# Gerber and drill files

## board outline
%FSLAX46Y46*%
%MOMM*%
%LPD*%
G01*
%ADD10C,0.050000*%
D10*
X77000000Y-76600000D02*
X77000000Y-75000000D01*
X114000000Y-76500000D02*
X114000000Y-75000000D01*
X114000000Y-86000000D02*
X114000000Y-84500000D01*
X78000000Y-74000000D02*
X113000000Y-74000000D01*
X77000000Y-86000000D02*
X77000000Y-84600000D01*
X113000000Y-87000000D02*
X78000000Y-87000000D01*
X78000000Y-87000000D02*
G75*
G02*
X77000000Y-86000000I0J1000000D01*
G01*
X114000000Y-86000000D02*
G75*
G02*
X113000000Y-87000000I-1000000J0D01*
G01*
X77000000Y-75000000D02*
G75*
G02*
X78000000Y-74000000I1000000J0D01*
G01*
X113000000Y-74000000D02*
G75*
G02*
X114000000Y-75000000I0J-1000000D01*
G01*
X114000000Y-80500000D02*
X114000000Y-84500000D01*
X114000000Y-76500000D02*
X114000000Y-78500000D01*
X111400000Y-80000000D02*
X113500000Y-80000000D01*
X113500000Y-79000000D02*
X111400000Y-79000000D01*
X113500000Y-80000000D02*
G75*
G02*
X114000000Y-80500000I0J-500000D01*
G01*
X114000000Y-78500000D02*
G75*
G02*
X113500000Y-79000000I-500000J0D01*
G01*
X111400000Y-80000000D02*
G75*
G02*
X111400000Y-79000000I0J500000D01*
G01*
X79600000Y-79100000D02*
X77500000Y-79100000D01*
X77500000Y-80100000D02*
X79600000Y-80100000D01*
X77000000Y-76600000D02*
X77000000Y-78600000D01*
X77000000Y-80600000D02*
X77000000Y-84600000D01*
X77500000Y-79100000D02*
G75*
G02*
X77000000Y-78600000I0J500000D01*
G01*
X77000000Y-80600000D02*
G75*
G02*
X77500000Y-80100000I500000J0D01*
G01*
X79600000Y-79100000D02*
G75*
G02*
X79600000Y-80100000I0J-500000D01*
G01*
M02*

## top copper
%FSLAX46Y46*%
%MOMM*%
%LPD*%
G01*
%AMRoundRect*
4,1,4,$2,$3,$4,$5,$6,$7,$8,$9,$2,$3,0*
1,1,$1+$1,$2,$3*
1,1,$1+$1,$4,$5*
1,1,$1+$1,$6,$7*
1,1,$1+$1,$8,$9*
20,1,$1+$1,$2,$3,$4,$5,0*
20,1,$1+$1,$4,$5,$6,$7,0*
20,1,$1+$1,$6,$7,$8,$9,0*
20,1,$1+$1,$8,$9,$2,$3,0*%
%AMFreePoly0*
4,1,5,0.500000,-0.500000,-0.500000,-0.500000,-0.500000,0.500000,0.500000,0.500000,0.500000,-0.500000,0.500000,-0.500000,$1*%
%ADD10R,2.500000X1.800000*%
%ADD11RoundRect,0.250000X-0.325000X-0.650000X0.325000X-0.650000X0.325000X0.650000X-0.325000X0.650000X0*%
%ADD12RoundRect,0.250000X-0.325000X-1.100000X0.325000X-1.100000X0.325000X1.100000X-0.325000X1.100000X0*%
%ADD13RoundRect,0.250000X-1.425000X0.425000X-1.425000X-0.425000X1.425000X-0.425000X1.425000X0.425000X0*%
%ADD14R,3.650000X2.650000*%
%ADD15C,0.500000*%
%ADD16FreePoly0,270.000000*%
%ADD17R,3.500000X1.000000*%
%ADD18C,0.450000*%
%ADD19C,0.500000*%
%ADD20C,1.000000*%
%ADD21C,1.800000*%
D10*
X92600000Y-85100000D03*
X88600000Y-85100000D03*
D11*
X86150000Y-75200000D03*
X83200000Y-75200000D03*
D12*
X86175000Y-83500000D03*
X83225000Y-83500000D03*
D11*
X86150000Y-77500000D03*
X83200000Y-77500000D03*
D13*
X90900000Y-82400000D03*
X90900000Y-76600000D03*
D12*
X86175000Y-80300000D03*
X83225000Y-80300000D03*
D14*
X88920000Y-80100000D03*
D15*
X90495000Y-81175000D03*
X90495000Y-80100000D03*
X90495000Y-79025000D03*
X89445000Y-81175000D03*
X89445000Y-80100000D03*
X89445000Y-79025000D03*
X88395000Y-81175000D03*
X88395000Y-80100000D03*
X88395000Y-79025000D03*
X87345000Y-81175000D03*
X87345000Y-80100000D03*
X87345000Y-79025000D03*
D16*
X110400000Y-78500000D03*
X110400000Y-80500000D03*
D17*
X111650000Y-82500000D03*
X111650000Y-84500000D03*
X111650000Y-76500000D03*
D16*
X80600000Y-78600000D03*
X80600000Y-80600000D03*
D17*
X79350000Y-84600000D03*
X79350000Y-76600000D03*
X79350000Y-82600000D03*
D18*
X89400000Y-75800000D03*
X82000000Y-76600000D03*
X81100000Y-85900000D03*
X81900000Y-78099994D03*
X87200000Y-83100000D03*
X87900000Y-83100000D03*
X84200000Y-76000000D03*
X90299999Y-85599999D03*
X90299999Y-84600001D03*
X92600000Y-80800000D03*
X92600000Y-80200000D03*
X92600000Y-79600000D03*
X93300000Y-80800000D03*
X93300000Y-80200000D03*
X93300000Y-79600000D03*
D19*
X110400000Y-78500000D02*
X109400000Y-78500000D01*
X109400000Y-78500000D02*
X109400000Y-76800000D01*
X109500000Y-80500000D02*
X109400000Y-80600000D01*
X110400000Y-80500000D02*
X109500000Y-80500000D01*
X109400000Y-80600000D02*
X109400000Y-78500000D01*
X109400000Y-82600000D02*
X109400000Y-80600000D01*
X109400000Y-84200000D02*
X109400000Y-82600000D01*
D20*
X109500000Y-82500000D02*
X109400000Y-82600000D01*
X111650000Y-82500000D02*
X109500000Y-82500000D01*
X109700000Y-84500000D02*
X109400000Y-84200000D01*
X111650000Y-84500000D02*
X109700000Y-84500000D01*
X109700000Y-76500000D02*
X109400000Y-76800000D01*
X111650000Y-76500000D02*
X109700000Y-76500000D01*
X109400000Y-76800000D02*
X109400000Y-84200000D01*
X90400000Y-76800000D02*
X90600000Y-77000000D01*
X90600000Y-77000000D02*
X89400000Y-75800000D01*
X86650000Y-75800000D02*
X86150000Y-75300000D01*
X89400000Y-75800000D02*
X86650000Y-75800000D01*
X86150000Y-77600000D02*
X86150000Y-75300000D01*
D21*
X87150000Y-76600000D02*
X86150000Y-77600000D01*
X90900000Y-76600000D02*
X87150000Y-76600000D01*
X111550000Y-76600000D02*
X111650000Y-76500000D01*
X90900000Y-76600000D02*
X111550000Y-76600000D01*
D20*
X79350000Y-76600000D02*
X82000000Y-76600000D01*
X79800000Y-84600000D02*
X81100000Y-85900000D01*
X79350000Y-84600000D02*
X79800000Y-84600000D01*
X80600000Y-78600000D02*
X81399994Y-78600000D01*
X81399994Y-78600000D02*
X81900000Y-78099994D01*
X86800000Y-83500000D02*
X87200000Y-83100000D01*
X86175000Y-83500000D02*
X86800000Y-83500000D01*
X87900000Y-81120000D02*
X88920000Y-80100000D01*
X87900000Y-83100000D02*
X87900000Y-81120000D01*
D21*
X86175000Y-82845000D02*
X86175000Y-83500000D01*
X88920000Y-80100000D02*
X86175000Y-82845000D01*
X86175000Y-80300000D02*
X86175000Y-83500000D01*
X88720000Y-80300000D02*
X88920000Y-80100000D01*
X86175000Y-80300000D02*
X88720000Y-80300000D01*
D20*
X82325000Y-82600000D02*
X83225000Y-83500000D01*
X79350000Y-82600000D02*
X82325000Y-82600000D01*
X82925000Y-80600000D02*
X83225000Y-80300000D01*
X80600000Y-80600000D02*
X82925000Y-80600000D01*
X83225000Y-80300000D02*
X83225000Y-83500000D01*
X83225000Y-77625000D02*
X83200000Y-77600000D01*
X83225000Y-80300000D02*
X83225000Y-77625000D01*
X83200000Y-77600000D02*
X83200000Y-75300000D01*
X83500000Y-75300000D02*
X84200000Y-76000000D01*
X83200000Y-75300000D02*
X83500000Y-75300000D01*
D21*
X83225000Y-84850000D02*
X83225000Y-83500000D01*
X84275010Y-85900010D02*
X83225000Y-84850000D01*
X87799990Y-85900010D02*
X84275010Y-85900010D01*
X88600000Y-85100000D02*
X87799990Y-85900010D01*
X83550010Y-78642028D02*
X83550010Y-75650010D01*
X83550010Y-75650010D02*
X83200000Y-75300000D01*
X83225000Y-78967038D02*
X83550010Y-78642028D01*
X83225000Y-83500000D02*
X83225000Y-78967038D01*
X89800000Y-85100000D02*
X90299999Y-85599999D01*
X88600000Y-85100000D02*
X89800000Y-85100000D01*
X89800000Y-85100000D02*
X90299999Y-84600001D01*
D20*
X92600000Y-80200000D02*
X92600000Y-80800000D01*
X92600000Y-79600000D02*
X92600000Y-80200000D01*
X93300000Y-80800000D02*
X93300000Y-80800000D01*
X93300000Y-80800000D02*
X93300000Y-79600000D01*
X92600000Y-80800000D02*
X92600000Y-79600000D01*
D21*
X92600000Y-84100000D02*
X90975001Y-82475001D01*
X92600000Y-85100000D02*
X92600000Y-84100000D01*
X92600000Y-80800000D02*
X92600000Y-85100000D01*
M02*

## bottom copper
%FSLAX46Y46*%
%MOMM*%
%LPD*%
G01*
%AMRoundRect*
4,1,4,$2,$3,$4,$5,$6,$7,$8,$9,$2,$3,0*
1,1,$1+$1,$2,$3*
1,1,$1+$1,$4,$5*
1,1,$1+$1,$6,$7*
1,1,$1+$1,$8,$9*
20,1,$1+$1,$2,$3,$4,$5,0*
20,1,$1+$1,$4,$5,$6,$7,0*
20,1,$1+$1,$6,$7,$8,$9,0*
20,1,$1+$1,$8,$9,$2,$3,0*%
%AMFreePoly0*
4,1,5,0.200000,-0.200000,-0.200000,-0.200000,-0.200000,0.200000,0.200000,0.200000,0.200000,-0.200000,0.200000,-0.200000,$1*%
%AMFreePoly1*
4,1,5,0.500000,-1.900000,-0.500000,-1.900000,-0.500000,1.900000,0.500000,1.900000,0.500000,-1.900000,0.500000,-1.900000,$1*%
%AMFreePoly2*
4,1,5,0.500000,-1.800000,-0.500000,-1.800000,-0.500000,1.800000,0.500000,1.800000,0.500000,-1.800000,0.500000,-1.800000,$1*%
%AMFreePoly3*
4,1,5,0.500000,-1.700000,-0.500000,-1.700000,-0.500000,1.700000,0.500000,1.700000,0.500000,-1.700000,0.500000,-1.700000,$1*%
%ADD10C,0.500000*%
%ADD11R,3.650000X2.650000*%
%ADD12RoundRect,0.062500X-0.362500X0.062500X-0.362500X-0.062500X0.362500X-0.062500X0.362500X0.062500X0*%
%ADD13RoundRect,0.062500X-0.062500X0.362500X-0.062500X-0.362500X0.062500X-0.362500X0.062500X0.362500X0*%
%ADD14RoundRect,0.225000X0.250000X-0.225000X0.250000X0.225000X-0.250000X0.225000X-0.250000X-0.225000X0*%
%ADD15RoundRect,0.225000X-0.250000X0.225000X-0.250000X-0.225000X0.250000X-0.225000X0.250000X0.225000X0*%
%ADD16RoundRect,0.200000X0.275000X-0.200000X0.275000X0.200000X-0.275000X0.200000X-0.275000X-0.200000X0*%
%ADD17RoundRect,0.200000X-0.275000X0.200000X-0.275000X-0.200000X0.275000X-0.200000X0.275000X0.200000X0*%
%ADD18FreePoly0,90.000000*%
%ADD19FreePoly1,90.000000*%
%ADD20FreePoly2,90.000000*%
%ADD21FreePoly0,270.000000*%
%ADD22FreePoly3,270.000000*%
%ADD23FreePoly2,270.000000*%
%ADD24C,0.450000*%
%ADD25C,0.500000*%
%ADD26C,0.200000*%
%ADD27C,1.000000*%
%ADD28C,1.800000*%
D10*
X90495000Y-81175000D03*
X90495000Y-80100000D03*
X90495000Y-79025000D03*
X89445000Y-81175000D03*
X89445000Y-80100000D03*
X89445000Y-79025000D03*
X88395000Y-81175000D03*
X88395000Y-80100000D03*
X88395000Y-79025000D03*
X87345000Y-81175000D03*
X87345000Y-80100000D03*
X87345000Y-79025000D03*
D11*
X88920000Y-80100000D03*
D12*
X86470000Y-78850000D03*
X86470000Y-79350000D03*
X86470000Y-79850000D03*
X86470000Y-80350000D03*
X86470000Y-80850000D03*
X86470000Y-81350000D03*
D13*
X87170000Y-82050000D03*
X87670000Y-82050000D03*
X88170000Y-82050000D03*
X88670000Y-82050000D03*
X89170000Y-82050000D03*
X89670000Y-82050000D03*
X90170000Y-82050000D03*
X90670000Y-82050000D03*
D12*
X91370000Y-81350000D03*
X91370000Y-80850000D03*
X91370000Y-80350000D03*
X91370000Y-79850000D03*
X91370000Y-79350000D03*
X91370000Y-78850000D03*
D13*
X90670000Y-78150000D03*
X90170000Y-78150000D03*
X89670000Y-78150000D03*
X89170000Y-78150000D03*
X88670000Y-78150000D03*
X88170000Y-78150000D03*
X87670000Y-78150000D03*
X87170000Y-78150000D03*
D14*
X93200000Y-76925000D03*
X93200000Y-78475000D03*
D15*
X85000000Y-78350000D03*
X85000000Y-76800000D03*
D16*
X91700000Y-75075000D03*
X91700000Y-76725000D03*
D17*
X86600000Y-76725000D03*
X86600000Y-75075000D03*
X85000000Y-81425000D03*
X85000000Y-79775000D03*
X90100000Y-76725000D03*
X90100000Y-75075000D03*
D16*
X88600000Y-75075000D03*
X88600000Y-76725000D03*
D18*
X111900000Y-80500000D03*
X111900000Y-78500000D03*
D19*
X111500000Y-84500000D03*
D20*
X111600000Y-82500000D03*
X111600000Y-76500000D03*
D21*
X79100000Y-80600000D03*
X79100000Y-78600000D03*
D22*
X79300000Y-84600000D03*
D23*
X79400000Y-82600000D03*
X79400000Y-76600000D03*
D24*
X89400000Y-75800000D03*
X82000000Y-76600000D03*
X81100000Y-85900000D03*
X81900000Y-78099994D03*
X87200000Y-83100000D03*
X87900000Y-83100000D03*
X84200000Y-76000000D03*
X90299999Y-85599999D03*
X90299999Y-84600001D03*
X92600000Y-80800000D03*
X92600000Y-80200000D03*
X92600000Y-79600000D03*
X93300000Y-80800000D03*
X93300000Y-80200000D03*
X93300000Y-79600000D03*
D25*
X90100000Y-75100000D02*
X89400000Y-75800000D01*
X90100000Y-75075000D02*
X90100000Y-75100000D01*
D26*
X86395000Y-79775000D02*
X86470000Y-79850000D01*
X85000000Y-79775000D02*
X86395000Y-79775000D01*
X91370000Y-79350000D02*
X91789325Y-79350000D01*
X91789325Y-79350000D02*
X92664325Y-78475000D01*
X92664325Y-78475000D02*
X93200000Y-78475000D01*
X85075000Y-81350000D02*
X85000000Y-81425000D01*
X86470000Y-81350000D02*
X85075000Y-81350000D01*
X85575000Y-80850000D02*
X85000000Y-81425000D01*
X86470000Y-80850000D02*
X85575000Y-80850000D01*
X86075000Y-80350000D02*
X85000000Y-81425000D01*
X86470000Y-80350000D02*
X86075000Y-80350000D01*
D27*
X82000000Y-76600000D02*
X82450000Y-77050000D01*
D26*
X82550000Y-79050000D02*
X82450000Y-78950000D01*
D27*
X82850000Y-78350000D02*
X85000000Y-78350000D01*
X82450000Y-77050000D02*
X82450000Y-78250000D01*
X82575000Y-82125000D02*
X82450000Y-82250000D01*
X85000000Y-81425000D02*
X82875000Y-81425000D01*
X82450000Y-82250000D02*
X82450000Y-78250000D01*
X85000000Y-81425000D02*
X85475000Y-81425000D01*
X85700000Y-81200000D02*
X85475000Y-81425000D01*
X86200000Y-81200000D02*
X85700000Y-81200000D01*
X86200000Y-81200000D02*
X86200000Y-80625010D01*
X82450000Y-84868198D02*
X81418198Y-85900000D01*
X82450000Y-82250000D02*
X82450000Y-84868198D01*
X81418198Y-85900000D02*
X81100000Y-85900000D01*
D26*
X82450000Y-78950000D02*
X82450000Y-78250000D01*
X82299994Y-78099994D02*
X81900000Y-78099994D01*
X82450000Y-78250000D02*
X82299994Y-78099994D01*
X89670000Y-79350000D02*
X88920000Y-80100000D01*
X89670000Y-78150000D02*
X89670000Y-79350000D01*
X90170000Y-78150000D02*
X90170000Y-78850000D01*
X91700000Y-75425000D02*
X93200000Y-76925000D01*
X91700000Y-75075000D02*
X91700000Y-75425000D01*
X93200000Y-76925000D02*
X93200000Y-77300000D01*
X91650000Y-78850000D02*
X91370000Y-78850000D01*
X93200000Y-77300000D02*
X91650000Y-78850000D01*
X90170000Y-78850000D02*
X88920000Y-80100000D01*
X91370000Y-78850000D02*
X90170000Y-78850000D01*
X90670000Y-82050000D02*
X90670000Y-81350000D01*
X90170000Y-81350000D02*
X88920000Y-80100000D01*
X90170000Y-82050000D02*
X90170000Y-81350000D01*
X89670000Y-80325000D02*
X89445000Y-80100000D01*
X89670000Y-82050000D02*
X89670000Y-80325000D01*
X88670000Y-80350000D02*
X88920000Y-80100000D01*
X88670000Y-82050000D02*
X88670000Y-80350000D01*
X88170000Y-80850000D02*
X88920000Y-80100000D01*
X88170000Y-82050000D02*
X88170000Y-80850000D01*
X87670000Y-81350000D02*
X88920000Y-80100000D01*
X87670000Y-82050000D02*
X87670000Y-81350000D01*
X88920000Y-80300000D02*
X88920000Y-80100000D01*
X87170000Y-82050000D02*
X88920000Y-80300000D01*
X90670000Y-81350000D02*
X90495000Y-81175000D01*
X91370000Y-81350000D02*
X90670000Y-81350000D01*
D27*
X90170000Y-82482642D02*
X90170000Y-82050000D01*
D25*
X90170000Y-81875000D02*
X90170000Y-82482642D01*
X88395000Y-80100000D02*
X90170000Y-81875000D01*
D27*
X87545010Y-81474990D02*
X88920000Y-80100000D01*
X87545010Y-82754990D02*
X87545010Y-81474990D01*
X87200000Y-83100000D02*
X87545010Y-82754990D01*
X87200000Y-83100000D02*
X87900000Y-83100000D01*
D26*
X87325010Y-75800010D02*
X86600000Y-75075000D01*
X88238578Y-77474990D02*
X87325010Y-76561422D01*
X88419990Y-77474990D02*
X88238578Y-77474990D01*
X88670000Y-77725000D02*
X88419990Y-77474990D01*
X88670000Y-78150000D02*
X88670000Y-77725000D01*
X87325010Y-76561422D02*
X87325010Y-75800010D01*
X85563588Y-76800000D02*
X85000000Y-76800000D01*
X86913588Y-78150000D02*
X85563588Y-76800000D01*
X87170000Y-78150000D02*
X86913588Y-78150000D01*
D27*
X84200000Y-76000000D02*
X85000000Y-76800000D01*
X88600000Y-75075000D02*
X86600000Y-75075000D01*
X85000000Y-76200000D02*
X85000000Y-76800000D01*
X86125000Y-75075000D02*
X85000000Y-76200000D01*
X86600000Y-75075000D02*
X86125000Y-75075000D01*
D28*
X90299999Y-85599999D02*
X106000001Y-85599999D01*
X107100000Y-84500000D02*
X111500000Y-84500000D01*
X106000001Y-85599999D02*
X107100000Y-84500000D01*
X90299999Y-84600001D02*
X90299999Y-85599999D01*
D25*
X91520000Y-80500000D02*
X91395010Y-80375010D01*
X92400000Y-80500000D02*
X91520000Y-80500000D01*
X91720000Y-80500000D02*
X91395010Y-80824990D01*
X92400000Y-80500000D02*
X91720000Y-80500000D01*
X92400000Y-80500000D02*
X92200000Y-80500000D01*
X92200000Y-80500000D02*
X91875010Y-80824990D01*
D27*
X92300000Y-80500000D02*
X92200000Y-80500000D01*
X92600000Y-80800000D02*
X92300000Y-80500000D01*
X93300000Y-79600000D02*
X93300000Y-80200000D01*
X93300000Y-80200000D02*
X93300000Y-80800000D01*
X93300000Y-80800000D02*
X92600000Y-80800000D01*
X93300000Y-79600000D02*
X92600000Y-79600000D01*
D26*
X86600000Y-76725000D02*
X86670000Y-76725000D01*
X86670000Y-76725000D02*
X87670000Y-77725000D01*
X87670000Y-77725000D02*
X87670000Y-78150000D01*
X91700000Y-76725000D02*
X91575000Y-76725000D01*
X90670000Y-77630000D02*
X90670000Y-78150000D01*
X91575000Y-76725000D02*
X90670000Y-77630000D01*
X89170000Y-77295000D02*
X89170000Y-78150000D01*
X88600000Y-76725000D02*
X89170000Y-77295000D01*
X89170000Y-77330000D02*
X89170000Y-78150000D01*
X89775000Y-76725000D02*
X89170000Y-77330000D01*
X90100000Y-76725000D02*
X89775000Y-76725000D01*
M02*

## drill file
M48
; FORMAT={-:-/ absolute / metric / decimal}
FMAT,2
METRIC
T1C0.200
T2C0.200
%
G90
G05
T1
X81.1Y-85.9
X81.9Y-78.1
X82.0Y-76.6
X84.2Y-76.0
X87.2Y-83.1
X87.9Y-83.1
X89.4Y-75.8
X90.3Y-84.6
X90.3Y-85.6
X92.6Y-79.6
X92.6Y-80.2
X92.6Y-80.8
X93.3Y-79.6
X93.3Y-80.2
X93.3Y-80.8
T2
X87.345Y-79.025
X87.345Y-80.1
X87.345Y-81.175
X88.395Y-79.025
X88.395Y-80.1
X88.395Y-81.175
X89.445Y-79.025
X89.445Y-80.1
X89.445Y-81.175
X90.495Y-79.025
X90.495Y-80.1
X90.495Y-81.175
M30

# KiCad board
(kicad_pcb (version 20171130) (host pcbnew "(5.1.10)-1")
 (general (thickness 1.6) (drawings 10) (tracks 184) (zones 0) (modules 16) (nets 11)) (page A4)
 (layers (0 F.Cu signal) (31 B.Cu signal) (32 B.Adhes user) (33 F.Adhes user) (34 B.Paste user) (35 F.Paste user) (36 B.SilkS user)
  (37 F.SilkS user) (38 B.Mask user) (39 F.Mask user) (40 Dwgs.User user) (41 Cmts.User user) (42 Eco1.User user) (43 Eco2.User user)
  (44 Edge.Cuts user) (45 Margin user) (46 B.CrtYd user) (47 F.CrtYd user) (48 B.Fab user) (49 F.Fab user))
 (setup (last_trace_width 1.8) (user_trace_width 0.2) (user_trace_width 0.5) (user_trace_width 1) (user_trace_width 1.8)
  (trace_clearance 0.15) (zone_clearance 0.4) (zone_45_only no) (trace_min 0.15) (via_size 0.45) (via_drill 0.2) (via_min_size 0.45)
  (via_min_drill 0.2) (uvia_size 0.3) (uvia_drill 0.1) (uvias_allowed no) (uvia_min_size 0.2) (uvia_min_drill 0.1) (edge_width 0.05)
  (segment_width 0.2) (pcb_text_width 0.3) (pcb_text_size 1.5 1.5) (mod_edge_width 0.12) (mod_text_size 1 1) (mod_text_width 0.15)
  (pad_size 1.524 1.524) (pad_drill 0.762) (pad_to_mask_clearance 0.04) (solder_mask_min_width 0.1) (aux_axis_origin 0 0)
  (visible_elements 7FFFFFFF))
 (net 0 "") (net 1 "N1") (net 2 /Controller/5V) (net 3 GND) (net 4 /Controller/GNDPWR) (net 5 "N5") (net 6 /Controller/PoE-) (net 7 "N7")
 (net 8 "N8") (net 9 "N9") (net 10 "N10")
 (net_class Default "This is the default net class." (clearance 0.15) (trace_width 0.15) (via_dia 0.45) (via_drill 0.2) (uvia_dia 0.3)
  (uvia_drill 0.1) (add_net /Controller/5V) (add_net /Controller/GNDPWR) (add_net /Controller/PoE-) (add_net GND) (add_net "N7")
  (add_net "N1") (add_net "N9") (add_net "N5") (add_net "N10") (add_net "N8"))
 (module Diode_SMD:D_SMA (layer F.Cu) (at 90.6 85.1)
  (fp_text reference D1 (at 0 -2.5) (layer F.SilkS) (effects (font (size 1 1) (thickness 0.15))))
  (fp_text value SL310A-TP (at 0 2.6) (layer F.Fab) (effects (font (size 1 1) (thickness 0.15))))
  (pad 2 smd rect (at 2 0) (size 2.5 1.8) (layers F.Cu F.Paste F.Mask) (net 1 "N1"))
  (pad 1 smd rect (at -2 0) (size 2.5 1.8) (layers F.Cu F.Paste F.Mask) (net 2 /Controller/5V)))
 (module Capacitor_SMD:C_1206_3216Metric (layer F.Cu) (at 84.675 75.2)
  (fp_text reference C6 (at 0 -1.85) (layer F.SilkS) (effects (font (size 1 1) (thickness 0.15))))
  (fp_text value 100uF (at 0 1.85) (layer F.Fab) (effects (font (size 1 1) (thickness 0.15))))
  (pad 2 smd roundrect (at 1.475 0) (size 1.15 1.8) (layers F.Cu F.Paste F.Mask) (roundrect_rratio 0.217391) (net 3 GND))
  (pad 1 smd roundrect (at -1.475 0) (size 1.15 1.8) (layers F.Cu F.Paste F.Mask) (roundrect_rratio 0.217391) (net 2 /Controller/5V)))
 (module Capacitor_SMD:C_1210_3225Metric (layer F.Cu) (at 84.7 83.5)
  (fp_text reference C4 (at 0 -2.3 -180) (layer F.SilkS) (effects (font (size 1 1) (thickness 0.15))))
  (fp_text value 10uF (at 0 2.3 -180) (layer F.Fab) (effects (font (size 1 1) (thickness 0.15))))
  (pad 2 smd roundrect (at 1.475 0) (size 1.15 2.7) (layers F.Cu F.Paste F.Mask) (roundrect_rratio 0.217391) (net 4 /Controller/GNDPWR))
  (pad 1 smd roundrect (at -1.475 0) (size 1.15 2.7) (layers F.Cu F.Paste F.Mask) (roundrect_rratio 0.217391) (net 2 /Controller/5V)))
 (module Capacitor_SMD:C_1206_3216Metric (layer F.Cu) (at 84.675 77.5)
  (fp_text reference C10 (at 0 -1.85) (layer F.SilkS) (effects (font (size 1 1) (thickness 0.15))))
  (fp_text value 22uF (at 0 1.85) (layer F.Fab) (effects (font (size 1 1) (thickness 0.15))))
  (pad 2 smd roundrect (at 1.475 0) (size 1.15 1.8) (layers F.Cu F.Paste F.Mask) (roundrect_rratio 0.217391) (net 3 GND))
  (pad 1 smd roundrect (at -1.475 0) (size 1.15 1.8) (layers F.Cu F.Paste F.Mask) (roundrect_rratio 0.217391) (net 2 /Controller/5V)))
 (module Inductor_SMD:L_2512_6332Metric (layer F.Cu) (at 90.9 79.5 270)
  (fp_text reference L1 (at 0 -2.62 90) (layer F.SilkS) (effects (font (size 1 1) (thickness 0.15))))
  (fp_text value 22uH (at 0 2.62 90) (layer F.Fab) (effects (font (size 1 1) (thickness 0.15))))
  (pad 2 smd roundrect (at 2.9 0 270) (size 1.35 3.35) (layers F.Cu F.Paste F.Mask) (roundrect_rratio 0.185185) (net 1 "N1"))
  (pad 1 smd roundrect (at -2.9 0 270) (size 1.35 3.35) (layers F.Cu F.Paste F.Mask) (roundrect_rratio 0.185185) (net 3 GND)))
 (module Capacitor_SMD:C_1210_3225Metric (layer F.Cu) (at 84.7 80.3)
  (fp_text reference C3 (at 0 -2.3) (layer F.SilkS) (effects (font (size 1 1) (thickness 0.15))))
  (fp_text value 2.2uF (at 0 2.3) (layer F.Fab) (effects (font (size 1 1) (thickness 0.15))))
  (pad 2 smd roundrect (at 1.475 0) (size 1.15 2.7) (layers F.Cu F.Paste F.Mask) (roundrect_rratio 0.217391) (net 4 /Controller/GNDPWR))
  (pad 1 smd roundrect (at -1.475 0) (size 1.15 2.7) (layers F.Cu F.Paste F.Mask) (roundrect_rratio 0.217391) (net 2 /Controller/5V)))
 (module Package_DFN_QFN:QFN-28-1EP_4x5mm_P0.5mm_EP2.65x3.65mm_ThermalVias (layer B.Cu) (at 88.92 80.1 270)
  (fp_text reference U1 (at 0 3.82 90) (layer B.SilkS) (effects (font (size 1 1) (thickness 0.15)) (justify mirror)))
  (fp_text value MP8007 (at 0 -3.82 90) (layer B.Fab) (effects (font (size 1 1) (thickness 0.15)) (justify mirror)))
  (pad "" smd roundrect (at 0.66 -1.22 270) (size 1.07 0.98) (layers B.Paste) (roundrect_rratio 0.25))
  (pad "" smd roundrect (at 0.66 0 270) (size 1.07 0.98) (layers B.Paste) (roundrect_rratio 0.25))
  (pad "" smd roundrect (at 0.66 1.22 270) (size 1.07 0.98) (layers B.Paste) (roundrect_rratio 0.25))
  (pad "" smd roundrect (at -0.66 -1.22 270) (size 1.07 0.98) (layers B.Paste) (roundrect_rratio 0.25))
  (pad "" smd roundrect (at -0.66 0 270) (size 1.07 0.98) (layers B.Paste) (roundrect_rratio 0.25))
  (pad "" smd roundrect (at -0.66 1.22 270) (size 1.07 0.98) (layers B.Paste) (roundrect_rratio 0.25))
  (pad 29 smd rect (at 0 0 270) (size 2.65 3.65) (layers F.Cu) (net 4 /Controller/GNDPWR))
  (pad 29 thru_hole circle (at 1.075 -1.575 270) (size 0.5 0.5) (drill 0.2) (layers *.Cu) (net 4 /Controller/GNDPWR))
  (pad 29 thru_hole circle (at 0 -1.575 270) (size 0.5 0.5) (drill 0.2) (layers *.Cu) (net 4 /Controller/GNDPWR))
  (pad 29 thru_hole circle (at -1.075 -1.575 270) (size 0.5 0.5) (drill 0.2) (layers *.Cu) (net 4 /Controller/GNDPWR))
  (pad 29 thru_hole circle (at 1.075 -0.525 270) (size 0.5 0.5) (drill 0.2) (layers *.Cu) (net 4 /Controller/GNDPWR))
  (pad 29 thru_hole circle (at 0 -0.525 270) (size 0.5 0.5) (drill 0.2) (layers *.Cu) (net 4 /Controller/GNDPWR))
  (pad 29 thru_hole circle (at -1.075 -0.525 270) (size 0.5 0.5) (drill 0.2) (layers *.Cu) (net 4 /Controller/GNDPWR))
  (pad 29 thru_hole circle (at 1.075 0.525 270) (size 0.5 0.5) (drill 0.2) (layers *.Cu) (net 4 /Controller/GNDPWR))
  (pad 29 thru_hole circle (at 0 0.525 270) (size 0.5 0.5) (drill 0.2) (layers *.Cu) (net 4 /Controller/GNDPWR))
  (pad 29 thru_hole circle (at -1.075 0.525 270) (size 0.5 0.5) (drill 0.2) (layers *.Cu) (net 4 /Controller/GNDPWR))
  (pad 29 thru_hole circle (at 1.075 1.575 270) (size 0.5 0.5) (drill 0.2) (layers *.Cu) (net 4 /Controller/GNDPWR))
  (pad 29 thru_hole circle (at 0 1.575 270) (size 0.5 0.5) (drill 0.2) (layers *.Cu) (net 4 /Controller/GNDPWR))
  (pad 29 thru_hole circle (at -1.075 1.575 270) (size 0.5 0.5) (drill 0.2) (layers *.Cu) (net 4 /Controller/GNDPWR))
  (pad 29 smd rect (at 0 0 270) (size 2.65 3.65) (layers B.Cu B.Mask) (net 4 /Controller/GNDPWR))
  (pad 28 smd roundrect (at -1.25 2.45 270) (size 0.25 0.85) (layers B.Cu B.Paste B.Mask) (roundrect_rratio 0.25))
  (pad 27 smd roundrect (at -0.75 2.45 270) (size 0.25 0.85) (layers B.Cu B.Paste B.Mask) (roundrect_rratio 0.25))
  (pad 26 smd roundrect (at -0.25 2.45 270) (size 0.25 0.85) (layers B.Cu B.Paste B.Mask) (roundrect_rratio 0.25) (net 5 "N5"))
  (pad 25 smd roundrect (at 0.25 2.45 270) (size 0.25 0.85) (layers B.Cu B.Paste B.Mask) (roundrect_rratio 0.25) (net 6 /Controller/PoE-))
  (pad 24 smd roundrect (at 0.75 2.45 270) (size 0.25 0.85) (layers B.Cu B.Paste B.Mask) (roundrect_rratio 0.25) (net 6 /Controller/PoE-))
  (pad 23 smd roundrect (at 1.25 2.45 270) (size 0.25 0.85) (layers B.Cu B.Paste B.Mask) (roundrect_rratio 0.25) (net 6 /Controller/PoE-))
  (pad 22 smd roundrect (at 1.95 1.75 270) (size 0.85 0.25) (layers B.Cu B.Paste B.Mask) (roundrect_rratio 0.25) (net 4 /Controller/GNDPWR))
  (pad 21 smd roundrect (at 1.95 1.25 270) (size 0.85 0.25) (layers B.Cu B.Paste B.Mask) (roundrect_rratio 0.25) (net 4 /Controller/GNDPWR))
  (pad 20 smd roundrect (at 1.95 0.75 270) (size 0.85 0.25) (layers B.Cu B.Paste B.Mask) (roundrect_rratio 0.25) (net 4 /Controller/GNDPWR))
  (pad 19 smd roundrect (at 1.95 0.25 270) (size 0.85 0.25) (layers B.Cu B.Paste B.Mask) (roundrect_rratio 0.25) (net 4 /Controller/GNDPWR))
  (pad 18 smd roundrect (at 1.95 -0.25 270) (size 0.85 0.25) (layers B.Cu B.Paste B.Mask) (roundrect_rratio 0.25))
  (pad 17 smd roundrect (at 1.95 -0.75 270) (size 0.85 0.25) (layers B.Cu B.Paste B.Mask) (roundrect_rratio 0.25) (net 4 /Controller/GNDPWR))
  (pad 16 smd roundrect (at 1.95 -1.25 270) (size 0.85 0.25) (layers B.Cu B.Paste B.Mask) (roundrect_rratio 0.25) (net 4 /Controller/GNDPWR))
  (pad 15 smd roundrect (at 1.95 -1.75 270) (size 0.85 0.25) (layers B.Cu B.Paste B.Mask) (roundrect_rratio 0.25) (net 4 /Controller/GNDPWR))
  (pad 14 smd roundrect (at 1.25 -2.45 270) (size 0.25 0.85) (layers B.Cu B.Paste B.Mask) (roundrect_rratio 0.25) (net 4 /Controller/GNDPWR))
  (pad 13 smd roundrect (at 0.75 -2.45 270) (size 0.25 0.85) (layers B.Cu B.Paste B.Mask) (roundrect_rratio 0.25) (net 1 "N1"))
  (pad 12 smd roundrect (at 0.25 -2.45 270) (size 0.25 0.85) (layers B.Cu B.Paste B.Mask) (roundrect_rratio 0.25) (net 1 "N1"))
  (pad 11 smd roundrect (at -0.25 -2.45 270) (size 0.25 0.85) (layers B.Cu B.Paste B.Mask) (roundrect_rratio 0.25))
  (pad 10 smd roundrect (at -0.75 -2.45 270) (size 0.25 0.85) (layers B.Cu B.Paste B.Mask) (roundrect_rratio 0.25) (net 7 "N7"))
  (pad 9 smd roundrect (at -1.25 -2.45 270) (size 0.25 0.85) (layers B.Cu B.Paste B.Mask) (roundrect_rratio 0.25) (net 4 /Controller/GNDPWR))
  (pad 8 smd roundrect (at -1.95 -1.75 270) (size 0.85 0.25) (layers B.Cu B.Paste B.Mask) (roundrect_rratio 0.25) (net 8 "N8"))
  (pad 7 smd roundrect (at -1.95 -1.25 270) (size 0.85 0.25) (layers B.Cu B.Paste B.Mask) (roundrect_rratio 0.25) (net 4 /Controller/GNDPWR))
  (pad 6 smd roundrect (at -1.95 -0.75 270) (size 0.85 0.25) (layers B.Cu B.Paste B.Mask) (roundrect_rratio 0.25) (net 4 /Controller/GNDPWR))
  (pad 5 smd roundrect (at -1.95 -0.25 270) (size 0.85 0.25) (layers B.Cu B.Paste B.Mask) (roundrect_rratio 0.25) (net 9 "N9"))
  (pad 4 smd roundrect (at -1.95 0.25 270) (size 0.85 0.25) (layers B.Cu B.Paste B.Mask) (roundrect_rratio 0.25) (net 2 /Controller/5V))
  (pad 3 smd roundrect (at -1.95 0.75 270) (size 0.85 0.25) (layers B.Cu B.Paste B.Mask) (roundrect_rratio 0.25))
  (pad 2 smd roundrect (at -1.95 1.25 270) (size 0.85 0.25) (layers B.Cu B.Paste B.Mask) (roundrect_rratio 0.25) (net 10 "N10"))
  (pad 1 smd roundrect (at -1.95 1.75 270) (size 0.85 0.25) (layers B.Cu B.Paste B.Mask) (roundrect_rratio 0.25) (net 2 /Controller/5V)))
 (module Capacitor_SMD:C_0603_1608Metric (layer B.Cu) (at 93.2 77.7 90)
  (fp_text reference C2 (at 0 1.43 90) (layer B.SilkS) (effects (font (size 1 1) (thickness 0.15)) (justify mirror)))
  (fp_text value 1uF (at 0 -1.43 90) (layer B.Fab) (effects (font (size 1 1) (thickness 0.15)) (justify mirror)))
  (pad 2 smd roundrect (at 0.775 0 90) (size 0.9 0.95) (layers B.Cu B.Paste B.Mask) (roundrect_rratio 0.25) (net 4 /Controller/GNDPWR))
  (pad 1 smd roundrect (at -0.775 0 90) (size 0.9 0.95) (layers B.Cu B.Paste B.Mask) (roundrect_rratio 0.25) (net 7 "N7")))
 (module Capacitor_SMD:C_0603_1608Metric (layer B.Cu) (at 85 77.575 270)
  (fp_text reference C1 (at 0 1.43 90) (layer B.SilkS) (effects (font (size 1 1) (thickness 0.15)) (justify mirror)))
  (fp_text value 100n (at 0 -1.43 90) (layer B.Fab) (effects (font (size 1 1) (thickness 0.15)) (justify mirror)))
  (pad 2 smd roundrect (at 0.775 0 270) (size 0.9 0.95) (layers B.Cu B.Paste B.Mask) (roundrect_rratio 0.25) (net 6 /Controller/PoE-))
  (pad 1 smd roundrect (at -0.775 0 270) (size 0.9 0.95) (layers B.Cu B.Paste B.Mask) (roundrect_rratio 0.25) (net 2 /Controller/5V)))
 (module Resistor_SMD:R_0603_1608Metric (layer B.Cu) (at 91.7 75.9 90)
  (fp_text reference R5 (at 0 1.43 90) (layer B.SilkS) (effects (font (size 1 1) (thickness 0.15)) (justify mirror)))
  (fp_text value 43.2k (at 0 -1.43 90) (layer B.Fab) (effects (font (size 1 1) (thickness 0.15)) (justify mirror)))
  (pad 2 smd roundrect (at 0.825 0 90) (size 0.8 0.95) (layers B.Cu B.Paste B.Mask) (roundrect_rratio 0.25) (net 4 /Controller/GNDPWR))
  (pad 1 smd roundrect (at -0.825 0 90) (size 0.8 0.95) (layers B.Cu B.Paste B.Mask) (roundrect_rratio 0.25) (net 8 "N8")))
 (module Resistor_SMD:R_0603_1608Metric (layer B.Cu) (at 86.6 75.9 270)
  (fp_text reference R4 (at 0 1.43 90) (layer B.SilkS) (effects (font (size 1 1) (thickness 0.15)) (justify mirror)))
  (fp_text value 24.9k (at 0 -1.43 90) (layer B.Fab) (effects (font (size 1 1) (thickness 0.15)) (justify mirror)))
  (pad 2 smd roundrect (at 0.825 0 270) (size 0.8 0.95) (layers B.Cu B.Paste B.Mask) (roundrect_rratio 0.25) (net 10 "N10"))
  (pad 1 smd roundrect (at -0.825 0 270) (size 0.8 0.95) (layers B.Cu B.Paste B.Mask) (roundrect_rratio 0.25) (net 2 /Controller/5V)))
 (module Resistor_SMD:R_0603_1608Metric (layer B.Cu) (at 85 80.6 270)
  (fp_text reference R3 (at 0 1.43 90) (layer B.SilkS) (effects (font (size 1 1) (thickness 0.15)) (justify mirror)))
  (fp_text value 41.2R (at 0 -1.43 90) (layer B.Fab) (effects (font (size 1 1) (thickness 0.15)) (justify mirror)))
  (pad 2 smd roundrect (at 0.825 0 270) (size 0.8 0.95) (layers B.Cu B.Paste B.Mask) (roundrect_rratio 0.25) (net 6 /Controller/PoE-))
  (pad 1 smd roundrect (at -0.825 0 270) (size 0.8 0.95) (layers B.Cu B.Paste B.Mask) (roundrect_rratio 0.25) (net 5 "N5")))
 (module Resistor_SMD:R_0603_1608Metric (layer B.Cu) (at 90.1 75.9 270)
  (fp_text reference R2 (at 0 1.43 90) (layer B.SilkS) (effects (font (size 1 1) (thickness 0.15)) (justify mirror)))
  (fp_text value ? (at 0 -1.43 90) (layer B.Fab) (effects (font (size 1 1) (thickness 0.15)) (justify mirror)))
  (pad 2 smd roundrect (at 0.825 0 270) (size 0.8 0.95) (layers B.Cu B.Paste B.Mask) (roundrect_rratio 0.25) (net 9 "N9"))
  (pad 1 smd roundrect (at -0.825 0 270) (size 0.8 0.95) (layers B.Cu B.Paste B.Mask) (roundrect_rratio 0.25) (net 3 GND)))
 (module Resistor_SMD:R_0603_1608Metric (layer B.Cu) (at 88.6 75.9 90)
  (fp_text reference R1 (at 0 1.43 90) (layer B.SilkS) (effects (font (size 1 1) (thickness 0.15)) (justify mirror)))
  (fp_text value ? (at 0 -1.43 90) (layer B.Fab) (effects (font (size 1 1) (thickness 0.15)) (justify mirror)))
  (pad 2 smd roundrect (at 0.825 0 90) (size 0.8 0.95) (layers B.Cu B.Paste B.Mask) (roundrect_rratio 0.25) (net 2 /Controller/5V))
  (pad 1 smd roundrect (at -0.825 0 90) (size 0.8 0.95) (layers B.Cu B.Paste B.Mask) (roundrect_rratio 0.25) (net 9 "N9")))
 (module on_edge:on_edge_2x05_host (layer F.Cu) (at 114 80.5 270)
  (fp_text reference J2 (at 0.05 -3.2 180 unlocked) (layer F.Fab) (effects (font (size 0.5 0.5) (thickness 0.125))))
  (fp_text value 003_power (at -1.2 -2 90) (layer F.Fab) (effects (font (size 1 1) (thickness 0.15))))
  (fp_line (start 0 0) (end 4 0) (layer Edge.Cuts) (width 0.05))
  (fp_line (start -4 0) (end -2 0) (layer Edge.Cuts) (width 0.05))
  (fp_line (start -0.5 2.6) (end -0.5 0.5) (layer Edge.Cuts) (width 0.05))
  (fp_line (start -1.5 0.5) (end -1.5 2.6) (layer Edge.Cuts) (width 0.05))
  (fp_arc (start 0 0.5) (end 0 0) (angle -90) (layer Edge.Cuts) (width 0.05))
  (fp_arc (start -2 0.5) (end -1.5 0.5) (angle -90) (layer Edge.Cuts) (width 0.05))
  (fp_arc (start -1 2.6) (end -1.5 2.6) (angle -180) (layer Edge.Cuts) (width 0.05))
  (pad 2 smd custom (at -2 3.6 270) (size 1 1) (layers F.Cu F.Mask) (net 3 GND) (zone_connect 0) (options (clearance outline) (anchor rect))
   (primitives))
  (pad 3 smd custom (at 0 3.6 270) (size 1 1) (layers F.Cu F.Mask) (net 3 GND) (zone_connect 0) (options (clearance outline) (anchor rect))
   (primitives))
  (pad 8 smd custom (at 0 2.1 90) (size 0.4 0.4) (layers B.Cu B.Mask) (zone_connect 0) (options (clearance outline) (anchor rect))
   (primitives))
  (pad 7 smd custom (at -2 2.1 90) (size 0.4 0.4) (layers B.Cu B.Mask) (zone_connect 0) (options (clearance outline) (anchor rect))
   (primitives))
  (pad 4 smd rect (at 2 2.35 270) (size 1 3.5) (layers F.Cu F.Mask) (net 3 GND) (zone_connect 0))
  (pad 10 smd custom (at 4 2.5 90) (size 1 3.8) (layers B.Cu B.Mask) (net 2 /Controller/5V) (zone_connect 0)
   (options (clearance outline) (anchor rect)) (primitives))
  (pad 9 smd custom (at 2 2.4 90) (size 1 3.6) (layers B.Cu B.Mask) (zone_connect 0) (options (clearance outline) (anchor rect))
   (primitives))
  (pad 6 smd custom (at -4 2.4 90) (size 1 3.6) (layers B.Cu B.Mask) (zone_connect 0) (options (clearance outline) (anchor rect))
   (primitives))
  (pad 5 smd rect (at 4 2.35 270) (size 1 3.5) (layers F.Cu F.Mask) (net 3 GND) (zone_connect 0))
  (pad 1 smd rect (at -4 2.35 270) (size 1 3.5) (layers F.Cu F.Mask) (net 3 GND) (zone_connect 0)))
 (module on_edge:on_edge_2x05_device (layer F.Cu) (at 77 80.6 270)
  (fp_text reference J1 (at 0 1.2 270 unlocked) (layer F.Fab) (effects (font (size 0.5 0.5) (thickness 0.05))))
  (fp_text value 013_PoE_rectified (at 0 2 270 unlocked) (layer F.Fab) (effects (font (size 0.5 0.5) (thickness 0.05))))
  (fp_line (start -1.5 -2.6) (end -1.5 -0.5) (layer Edge.Cuts) (width 0.05))
  (fp_line (start -0.5 -0.5) (end -0.5 -2.6) (layer Edge.Cuts) (width 0.05))
  (fp_line (start -4 0) (end -2 0) (layer Edge.Cuts) (width 0.05))
  (fp_line (start 0 0) (end 4 0) (layer Edge.Cuts) (width 0.05))
  (fp_arc (start -2 -0.5) (end -2 0) (angle -90) (layer Edge.Cuts) (width 0.05))
  (fp_arc (start 0 -0.5) (end -0.5 -0.5) (angle -90) (layer Edge.Cuts) (width 0.05))
  (fp_arc (start -1 -2.6) (end -0.5 -2.6) (angle -180) (layer Edge.Cuts) (width 0.05))
  (pad 2 smd custom (at -2 -3.6 270) (size 1 1) (layers F.Cu F.Mask) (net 6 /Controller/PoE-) (zone_connect 0)
   (options (clearance outline) (anchor rect)) (primitives))
  (pad 3 smd custom (at 0 -3.6 270) (size 1 1) (layers F.Cu F.Mask) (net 2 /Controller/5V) (zone_connect 0)
   (options (clearance outline) (anchor rect)) (primitives))
  (pad 8 smd custom (at 0 -2.1 270) (size 0.4 0.4) (layers B.Cu B.Mask) (zone_connect 0) (options (clearance outline) (anchor rect))
   (primitives))
  (pad 7 smd custom (at -2 -2.1 270) (size 0.4 0.4) (layers B.Cu B.Mask) (zone_connect 0) (options (clearance outline) (anchor rect))
   (primitives))
  (pad 10 smd custom (at 4 -2.3 270) (size 1 3.4) (layers B.Cu B.Mask) (zone_connect 0) (options (clearance outline) (anchor rect))
   (primitives))
  (pad 9 smd custom (at 2 -2.4 270) (size 1 3.6) (layers B.Cu B.Mask) (zone_connect 0) (options (clearance outline) (anchor rect))
   (primitives))
  (pad 6 smd custom (at -4 -2.4 270) (size 1 3.6) (layers B.Cu B.Mask) (zone_connect 0) (options (clearance outline) (anchor rect))
   (primitives))
  (pad 5 smd rect (at 4 -2.35 90) (size 1 3.5) (layers F.Cu F.Mask) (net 6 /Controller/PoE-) (zone_connect 0))
  (pad 1 smd rect (at -4 -2.35 90) (size 1 3.5) (layers F.Cu F.Mask) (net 6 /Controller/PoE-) (zone_connect 0))
  (pad 4 smd rect (at 2 -2.35 90) (size 1 3.5) (layers F.Cu F.Mask) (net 2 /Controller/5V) (zone_connect 0)))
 (gr_line (start 77 76.6) (end 77 75) (layer Edge.Cuts) (width 0.05))
 (gr_line (start 114 76.5) (end 114 75) (layer Edge.Cuts) (width 0.05))
 (gr_line (start 114 86) (end 114 84.5) (layer Edge.Cuts) (width 0.05))
 (gr_line (start 78 74) (end 113 74) (layer Edge.Cuts) (width 0.05))
 (gr_line (start 77 86) (end 77 84.6) (layer Edge.Cuts) (width 0.05))
 (gr_line (start 113 87) (end 78 87) (layer Edge.Cuts) (width 0.05))
 (gr_arc (start 78 86) (end 77 86) (angle -90) (layer Edge.Cuts) (width 0.05))
 (gr_arc (start 113 86) (end 113 87) (angle -90) (layer Edge.Cuts) (width 0.05))
 (gr_arc (start 78 75) (end 78 74) (angle -90) (layer Edge.Cuts) (width 0.05))
 (gr_arc (start 113 75) (end 114 75) (angle -90) (layer Edge.Cuts) (width 0.05))
 (segment (start 110.4 78.5) (end 109.4 78.5) (width 0.5) (layer F.Cu) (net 3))
 (segment (start 109.4 78.5) (end 109.4 76.8) (width 0.5) (layer F.Cu) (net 3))
 (segment (start 109.5 80.5) (end 109.4 80.6) (width 0.5) (layer F.Cu) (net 3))
 (segment (start 110.4 80.5) (end 109.5 80.5) (width 0.5) (layer F.Cu) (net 3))
 (segment (start 109.4 80.6) (end 109.4 78.5) (width 0.5) (layer F.Cu) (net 3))
 (segment (start 109.4 82.6) (end 109.4 80.6) (width 0.5) (layer F.Cu) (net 3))
 (segment (start 109.4 84.2) (end 109.4 82.6) (width 0.5) (layer F.Cu) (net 3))
 (segment (start 109.5 82.5) (end 109.4 82.6) (width 1) (layer F.Cu) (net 3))
 (segment (start 111.65 82.5) (end 109.5 82.5) (width 1) (layer F.Cu) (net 3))
 (segment (start 109.7 84.5) (end 109.4 84.2) (width 1) (layer F.Cu) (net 3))
 (segment (start 111.65 84.5) (end 109.7 84.5) (width 1) (layer F.Cu) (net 3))
 (segment (start 109.7 76.5) (end 109.4 76.8) (width 1) (layer F.Cu) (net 3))
 (segment (start 111.65 76.5) (end 109.7 76.5) (width 1) (layer F.Cu) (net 3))
 (segment (start 109.4 76.8) (end 109.4 84.2) (width 1) (layer F.Cu) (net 3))
 (via (at 89.4 75.8) (size 0.45) (drill 0.2) (layers F.Cu B.Cu) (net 3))
 (segment (start 90.1 75.1) (end 89.4 75.8) (width 0.5) (layer B.Cu) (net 3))
 (segment (start 90.1 75.075) (end 90.1 75.1) (width 0.5) (layer B.Cu) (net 3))
 (segment (start 90.4 76.8) (end 90.6 77) (width 1) (layer F.Cu) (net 3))
 (segment (start 90.6 77) (end 89.4 75.8) (width 1) (layer F.Cu) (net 3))
 (segment (start 86.65 75.8) (end 86.15 75.3) (width 1) (layer F.Cu) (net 3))
 (segment (start 89.4 75.8) (end 86.65 75.8) (width 1) (layer F.Cu) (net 3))
 (segment (start 86.15 77.6) (end 86.15 75.3) (width 1) (layer F.Cu) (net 3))
 (segment (start 87.15 76.6) (end 86.15 77.6) (width 1.8) (layer F.Cu) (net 3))
 (segment (start 90.9 76.6) (end 87.15 76.6) (width 1.8) (layer F.Cu) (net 3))
 (segment (start 111.55 76.6) (end 111.65 76.5) (width 1.8) (layer F.Cu) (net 3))
 (segment (start 90.9 76.6) (end 111.55 76.6) (width 1.8) (layer F.Cu) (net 3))
 (segment (start 86.395 79.775) (end 86.47 79.85) (width 0.2) (layer B.Cu) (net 5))
 (segment (start 85 79.775) (end 86.395 79.775) (width 0.2) (layer B.Cu) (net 5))
 (segment (start 91.37 79.35) (end 91.789325 79.35) (width 0.2) (layer B.Cu) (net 7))
 (segment (start 91.789325 79.35) (end 92.664325 78.475) (width 0.2) (layer B.Cu) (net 7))
 (segment (start 92.664325 78.475) (end 93.2 78.475) (width 0.2) (layer B.Cu) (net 7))
 (segment (start 85.075 81.35) (end 85 81.425) (width 0.2) (layer B.Cu) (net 6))
 (segment (start 86.47 81.35) (end 85.075 81.35) (width 0.2) (layer B.Cu) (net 6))
 (segment (start 85.575 80.85) (end 85 81.425) (width 0.2) (layer B.Cu) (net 6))
 (segment (start 86.47 80.85) (end 85.575 80.85) (width 0.2) (layer B.Cu) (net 6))
 (segment (start 86.075 80.35) (end 85 81.425) (width 0.2) (layer B.Cu) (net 6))
 (segment (start 86.47 80.35) (end 86.075 80.35) (width 0.2) (layer B.Cu) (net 6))
 (via (at 82 76.6) (size 0.45) (drill 0.2) (layers F.Cu B.Cu) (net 6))
 (segment (start 79.35 76.6) (end 82 76.6) (width 1) (layer F.Cu) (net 6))
 (segment (start 82 76.6) (end 82.45 77.05) (width 1) (layer B.Cu) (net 6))
 (segment (start 82.55 79.05) (end 82.45 78.95) (width 0.2) (layer B.Cu) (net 6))
 (segment (start 82.85 78.35) (end 85 78.35) (width 1) (layer B.Cu) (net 6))
 (segment (start 82.45 77.05) (end 82.45 78.25) (width 1) (layer B.Cu) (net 6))
 (segment (start 82.575 82.125) (end 82.45 82.25) (width 1) (layer B.Cu) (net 6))
 (segment (start 85 81.425) (end 82.875 81.425) (width 1) (layer B.Cu) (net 6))
 (segment (start 82.45 82.25) (end 82.45 78.25) (width 1) (layer B.Cu) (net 6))
 (segment (start 85 81.425) (end 85.475 81.425) (width 1) (layer B.Cu) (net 6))
 (segment (start 85.7 81.2) (end 85.475 81.425) (width 1) (layer B.Cu) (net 6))
 (segment (start 86.2 81.2) (end 85.7 81.2) (width 1) (layer B.Cu) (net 6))
 (segment (start 86.2 81.2) (end 86.2 80.62501) (width 1) (layer B.Cu) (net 6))
 (segment (start 82.45 84.868198) (end 81.418198 85.9) (width 1) (layer B.Cu) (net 6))
 (segment (start 82.45 82.25) (end 82.45 84.868198) (width 1) (layer B.Cu) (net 6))
 (segment (start 79.8 84.6) (end 81.1 85.9) (width 1) (layer F.Cu) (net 6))
 (segment (start 79.35 84.6) (end 79.8 84.6) (width 1) (layer F.Cu) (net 6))
 (segment (start 81.418198 85.9) (end 81.1 85.9) (width 1) (layer B.Cu) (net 6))
 (via (at 81.1 85.9) (size 0.45) (drill 0.2) (layers F.Cu B.Cu) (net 6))
 (via (at 81.9 78.099994) (size 0.45) (drill 0.2) (layers F.Cu B.Cu) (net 6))
 (segment (start 82.45 78.95) (end 82.45 78.25) (width 0.2) (layer B.Cu) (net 6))
 (segment (start 82.299994 78.099994) (end 81.9 78.099994) (width 0.2) (layer B.Cu) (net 6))
 (segment (start 82.45 78.25) (end 82.299994 78.099994) (width 0.2) (layer B.Cu) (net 6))
 (segment (start 80.6 78.6) (end 81.399994 78.6) (width 1) (layer F.Cu) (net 6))
 (segment (start 81.399994 78.6) (end 81.9 78.099994) (width 1) (layer F.Cu) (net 6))
 (segment (start 89.67 79.35) (end 88.92 80.1) (width 0.2) (layer B.Cu) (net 4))
 (segment (start 89.67 78.15) (end 89.67 79.35) (width 0.2) (layer B.Cu) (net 4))
 (segment (start 90.17 78.15) (end 90.17 78.85) (width 0.2) (layer B.Cu) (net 4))
 (segment (start 91.7 75.425) (end 93.2 76.925) (width 0.2) (layer B.Cu) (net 4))
 (segment (start 91.7 75.075) (end 91.7 75.425) (width 0.2) (layer B.Cu) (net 4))
 (segment (start 93.2 76.925) (end 93.2 77.3) (width 0.2) (layer B.Cu) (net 4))
 (segment (start 91.65 78.85) (end 91.37 78.85) (width 0.2) (layer B.Cu) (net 4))
 (segment (start 93.2 77.3) (end 91.65 78.85) (width 0.2) (layer B.Cu) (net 4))
 (segment (start 90.17 78.85) (end 88.92 80.1) (width 0.2) (layer B.Cu) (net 4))
 (segment (start 91.37 78.85) (end 90.17 78.85) (width 0.2) (layer B.Cu) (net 4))
 (segment (start 90.67 82.05) (end 90.67 81.35) (width 0.2) (layer B.Cu) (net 4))
 (segment (start 90.17 81.35) (end 88.92 80.1) (width 0.2) (layer B.Cu) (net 4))
 (segment (start 90.17 82.05) (end 90.17 81.35) (width 0.2) (layer B.Cu) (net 4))
 (segment (start 89.67 80.325) (end 89.445 80.1) (width 0.2) (layer B.Cu) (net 4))
 (segment (start 89.67 82.05) (end 89.67 80.325) (width 0.2) (layer B.Cu) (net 4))
 (segment (start 88.67 80.35) (end 88.92 80.1) (width 0.2) (layer B.Cu) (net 4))
 (segment (start 88.67 82.05) (end 88.67 80.35) (width 0.2) (layer B.Cu) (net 4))
 (segment (start 88.17 80.85) (end 88.92 80.1) (width 0.2) (layer B.Cu) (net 4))
 (segment (start 88.17 82.05) (end 88.17 80.85) (width 0.2) (layer B.Cu) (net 4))
 (segment (start 87.67 81.35) (end 88.92 80.1) (width 0.2) (layer B.Cu) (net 4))
 (segment (start 87.67 82.05) (end 87.67 81.35) (width 0.2) (layer B.Cu) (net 4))
 (segment (start 88.92 80.3) (end 88.92 80.1) (width 0.2) (layer B.Cu) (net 4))
 (segment (start 87.17 82.05) (end 88.92 80.3) (width 0.2) (layer B.Cu) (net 4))
 (segment (start 90.67 81.35) (end 90.495 81.175) (width 0.2) (layer B.Cu) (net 4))
 (segment (start 91.37 81.35) (end 90.67 81.35) (width 0.2) (layer B.Cu) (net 4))
 (segment (start 90.17 82.482642) (end 90.17 82.05) (width 1) (layer B.Cu) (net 4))
 (segment (start 90.17 81.875) (end 90.17 82.482642) (width 0.5) (layer B.Cu) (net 4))
 (segment (start 88.395 80.1) (end 90.17 81.875) (width 0.5) (layer B.Cu) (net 4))
 (via (at 87.2 83.1) (size 0.45) (drill 0.2) (layers F.Cu B.Cu) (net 4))
 (segment (start 86.8 83.5) (end 87.2 83.1) (width 1) (layer F.Cu) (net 4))
 (segment (start 86.175 83.5) (end 86.8 83.5) (width 1) (layer F.Cu) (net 4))
 (segment (start 87.54501 81.47499) (end 88.92 80.1) (width 1) (layer B.Cu) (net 4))
 (segment (start 87.54501 82.75499) (end 87.54501 81.47499) (width 1) (layer B.Cu) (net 4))
 (segment (start 87.2 83.1) (end 87.54501 82.75499) (width 1) (layer B.Cu) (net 4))
 (via (at 87.9 83.1) (size 0.45) (drill 0.2) (layers F.Cu B.Cu) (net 4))
 (segment (start 87.2 83.1) (end 87.9 83.1) (width 1) (layer B.Cu) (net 4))
 (segment (start 87.9 81.12) (end 88.92 80.1) (width 1) (layer F.Cu) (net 4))
 (segment (start 87.9 83.1) (end 87.9 81.12) (width 1) (layer F.Cu) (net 4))
 (segment (start 86.175 82.845) (end 86.175 83.5) (width 1.8) (layer F.Cu) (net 4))
 (segment (start 88.92 80.1) (end 86.175 82.845) (width 1.8) (layer F.Cu) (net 4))
 (segment (start 86.175 80.3) (end 86.175 83.5) (width 1.8) (layer F.Cu) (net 4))
 (segment (start 88.72 80.3) (end 88.92 80.1) (width 1.8) (layer F.Cu) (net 4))
 (segment (start 86.175 80.3) (end 88.72 80.3) (width 1.8) (layer F.Cu) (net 4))
 (segment (start 87.32501 75.80001) (end 86.6 75.075) (width 0.2) (layer B.Cu) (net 2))
 (segment (start 88.238578 77.47499) (end 87.32501 76.561422) (width 0.2) (layer B.Cu) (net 2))
 (segment (start 88.41999 77.47499) (end 88.238578 77.47499) (width 0.2) (layer B.Cu) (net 2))
 (segment (start 88.67 77.725) (end 88.41999 77.47499) (width 0.2) (layer B.Cu) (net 2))
 (segment (start 88.67 78.15) (end 88.67 77.725) (width 0.2) (layer B.Cu) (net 2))
 (segment (start 87.32501 76.561422) (end 87.32501 75.80001) (width 0.2) (layer B.Cu) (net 2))
 (segment (start 85.563588 76.8) (end 85 76.8) (width 0.2) (layer B.Cu) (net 2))
 (segment (start 86.913588 78.15) (end 85.563588 76.8) (width 0.2) (layer B.Cu) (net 2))
 (segment (start 87.17 78.15) (end 86.913588 78.15) (width 0.2) (layer B.Cu) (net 2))
 (segment (start 82.325 82.6) (end 83.225 83.5) (width 1) (layer F.Cu) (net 2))
 (segment (start 79.35 82.6) (end 82.325 82.6) (width 1) (layer F.Cu) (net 2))
 (segment (start 82.925 80.6) (end 83.225 80.3) (width 1) (layer F.Cu) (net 2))
 (segment (start 80.6 80.6) (end 82.925 80.6) (width 1) (layer F.Cu) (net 2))
 (segment (start 83.225 80.3) (end 83.225 83.5) (width 1) (layer F.Cu) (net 2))
 (segment (start 83.225 77.625) (end 83.2 77.6) (width 1) (layer F.Cu) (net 2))
 (segment (start 83.225 80.3) (end 83.225 77.625) (width 1) (layer F.Cu) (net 2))
 (segment (start 83.2 77.6) (end 83.2 75.3) (width 1) (layer F.Cu) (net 2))
 (via (at 84.2 76) (size 0.45) (drill 0.2) (layers F.Cu B.Cu) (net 2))
 (segment (start 83.5 75.3) (end 84.2 76) (width 1) (layer F.Cu) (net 2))
 (segment (start 83.2 75.3) (end 83.5 75.3) (width 1) (layer F.Cu) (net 2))
 (segment (start 84.2 76) (end 85 76.8) (width 1) (layer B.Cu) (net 2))
 (segment (start 88.6 75.075) (end 86.6 75.075) (width 1) (layer B.Cu) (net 2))
 (segment (start 85 76.2) (end 85 76.8) (width 1) (layer B.Cu) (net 2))
 (segment (start 86.125 75.075) (end 85 76.2) (width 1) (layer B.Cu) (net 2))
 (segment (start 86.6 75.075) (end 86.125 75.075) (width 1) (layer B.Cu) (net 2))
 (segment (start 83.225 84.85) (end 83.225 83.5) (width 1.8) (layer F.Cu) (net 2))
 (segment (start 84.27501 85.90001) (end 83.225 84.85) (width 1.8) (layer F.Cu) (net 2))
 (segment (start 87.79999 85.90001) (end 84.27501 85.90001) (width 1.8) (layer F.Cu) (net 2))
 (segment (start 88.6 85.1) (end 87.79999 85.90001) (width 1.8) (layer F.Cu) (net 2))
 (segment (start 83.55001 78.642028) (end 83.55001 75.65001) (width 1.8) (layer F.Cu) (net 2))
 (segment (start 83.55001 75.65001) (end 83.2 75.3) (width 1.8) (layer F.Cu) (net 2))
 (segment (start 83.225 78.967038) (end 83.55001 78.642028) (width 1.8) (layer F.Cu) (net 2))
 (segment (start 83.225 83.5) (end 83.225 78.967038) (width 1.8) (layer F.Cu) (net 2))
 (via (at 90.299999 85.599999) (size 0.45) (drill 0.2) (layers F.Cu B.Cu) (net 2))
 (segment (start 89.8 85.1) (end 90.299999 85.599999) (width 1.8) (layer F.Cu) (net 2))
 (segment (start 88.6 85.1) (end 89.8 85.1) (width 1.8) (layer F.Cu) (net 2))
 (segment (start 90.299999 85.599999) (end 106.000001 85.599999) (width 1.8) (layer B.Cu) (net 2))
 (segment (start 107.1 84.5) (end 111.5 84.5) (width 1.8) (layer B.Cu) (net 2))
 (segment (start 106.000001 85.599999) (end 107.1 84.5) (width 1.8) (layer B.Cu) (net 2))
 (via (at 90.299999 84.600001) (size 0.45) (drill 0.2) (layers F.Cu B.Cu) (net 2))
 (segment (start 89.8 85.1) (end 90.299999 84.600001) (width 1.8) (layer F.Cu) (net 2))
 (segment (start 90.299999 84.600001) (end 90.299999 85.599999) (width 1.8) (layer B.Cu) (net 2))
 (segment (start 91.52 80.5) (end 91.39501 80.37501) (width 0.5) (layer B.Cu) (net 1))
 (segment (start 92.4 80.5) (end 91.52 80.5) (width 0.5) (layer B.Cu) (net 1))
 (segment (start 91.72 80.5) (end 91.39501 80.82499) (width 0.5) (layer B.Cu) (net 1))
 (segment (start 92.4 80.5) (end 91.72 80.5) (width 0.5) (layer B.Cu) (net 1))
 (segment (start 92.4 80.5) (end 92.2 80.5) (width 0.5) (layer B.Cu) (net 1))
 (segment (start 92.2 80.5) (end 91.87501 80.82499) (width 0.5) (layer B.Cu) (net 1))
 (via (at 92.6 80.8) (size 0.45) (drill 0.2) (layers F.Cu B.Cu) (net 1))
 (segment (start 92.3 80.5) (end 92.2 80.5) (width 1) (layer B.Cu) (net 1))
 (segment (start 92.6 80.8) (end 92.3 80.5) (width 1) (layer B.Cu) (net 1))
 (segment (start 92.6 80.2) (end 92.6 80.8) (width 1) (layer F.Cu) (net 1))
 (via (at 92.6 80.2) (size 0.45) (drill 0.2) (layers F.Cu B.Cu) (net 1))
 (segment (start 92.6 79.6) (end 92.6 80.2) (width 1) (layer F.Cu) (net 1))
 (via (at 92.6 79.6) (size 0.45) (drill 0.2) (layers F.Cu B.Cu) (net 1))
 (segment (start 93.3 80.8) (end 93.3 80.8) (width 1) (layer F.Cu) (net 1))
 (via (at 93.3 80.8) (size 0.45) (drill 0.2) (layers F.Cu B.Cu) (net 1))
 (via (at 93.3 80.2) (size 0.45) (drill 0.2) (layers F.Cu B.Cu) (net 1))
 (via (at 93.3 79.6) (size 0.45) (drill 0.2) (layers F.Cu B.Cu) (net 1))
 (segment (start 93.3 79.6) (end 93.3 80.2) (width 1) (layer B.Cu) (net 1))
 (segment (start 93.3 80.2) (end 93.3 80.8) (width 1) (layer B.Cu) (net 1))
 (segment (start 93.3 80.8) (end 92.6 80.8) (width 1) (layer B.Cu) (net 1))
 (segment (start 93.3 79.6) (end 92.6 79.6) (width 1) (layer B.Cu) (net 1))
 (segment (start 93.3 80.8) (end 93.3 79.6) (width 1) (layer F.Cu) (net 1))
 (segment (start 92.6 80.8) (end 92.6 79.6) (width 1) (layer F.Cu) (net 1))
 (segment (start 92.6 84.1) (end 90.975001 82.475001) (width 1.8) (layer F.Cu) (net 1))
 (segment (start 92.6 85.1) (end 92.6 84.1) (width 1.8) (layer F.Cu) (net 1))
 (segment (start 92.6 80.8) (end 92.6 85.1) (width 1.8) (layer F.Cu) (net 1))
 (segment (start 86.6 76.725) (end 86.67 76.725) (width 0.2) (layer B.Cu) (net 10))
 (segment (start 86.67 76.725) (end 87.67 77.725) (width 0.2) (layer B.Cu) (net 10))
 (segment (start 87.67 77.725) (end 87.67 78.15) (width 0.2) (layer B.Cu) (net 10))
 (segment (start 91.7 76.725) (end 91.575 76.725) (width 0.2) (layer B.Cu) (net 8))
 (segment (start 90.67 77.63) (end 90.67 78.15) (width 0.2) (layer B.Cu) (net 8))
 (segment (start 91.575 76.725) (end 90.67 77.63) (width 0.2) (layer B.Cu) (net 8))
 (segment (start 89.17 77.295) (end 89.17 78.15) (width 0.2) (layer B.Cu) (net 9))
 (segment (start 88.6 76.725) (end 89.17 77.295) (width 0.2) (layer B.Cu) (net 9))
 (segment (start 89.17 77.33) (end 89.17 78.15) (width 0.2) (layer B.Cu) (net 9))
 (segment (start 89.775 76.725) (end 89.17 77.33) (width 0.2) (layer B.Cu) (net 9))
 (segment (start 90.1 76.725) (end 89.775 76.725) (width 0.2) (layer B.Cu) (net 9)))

